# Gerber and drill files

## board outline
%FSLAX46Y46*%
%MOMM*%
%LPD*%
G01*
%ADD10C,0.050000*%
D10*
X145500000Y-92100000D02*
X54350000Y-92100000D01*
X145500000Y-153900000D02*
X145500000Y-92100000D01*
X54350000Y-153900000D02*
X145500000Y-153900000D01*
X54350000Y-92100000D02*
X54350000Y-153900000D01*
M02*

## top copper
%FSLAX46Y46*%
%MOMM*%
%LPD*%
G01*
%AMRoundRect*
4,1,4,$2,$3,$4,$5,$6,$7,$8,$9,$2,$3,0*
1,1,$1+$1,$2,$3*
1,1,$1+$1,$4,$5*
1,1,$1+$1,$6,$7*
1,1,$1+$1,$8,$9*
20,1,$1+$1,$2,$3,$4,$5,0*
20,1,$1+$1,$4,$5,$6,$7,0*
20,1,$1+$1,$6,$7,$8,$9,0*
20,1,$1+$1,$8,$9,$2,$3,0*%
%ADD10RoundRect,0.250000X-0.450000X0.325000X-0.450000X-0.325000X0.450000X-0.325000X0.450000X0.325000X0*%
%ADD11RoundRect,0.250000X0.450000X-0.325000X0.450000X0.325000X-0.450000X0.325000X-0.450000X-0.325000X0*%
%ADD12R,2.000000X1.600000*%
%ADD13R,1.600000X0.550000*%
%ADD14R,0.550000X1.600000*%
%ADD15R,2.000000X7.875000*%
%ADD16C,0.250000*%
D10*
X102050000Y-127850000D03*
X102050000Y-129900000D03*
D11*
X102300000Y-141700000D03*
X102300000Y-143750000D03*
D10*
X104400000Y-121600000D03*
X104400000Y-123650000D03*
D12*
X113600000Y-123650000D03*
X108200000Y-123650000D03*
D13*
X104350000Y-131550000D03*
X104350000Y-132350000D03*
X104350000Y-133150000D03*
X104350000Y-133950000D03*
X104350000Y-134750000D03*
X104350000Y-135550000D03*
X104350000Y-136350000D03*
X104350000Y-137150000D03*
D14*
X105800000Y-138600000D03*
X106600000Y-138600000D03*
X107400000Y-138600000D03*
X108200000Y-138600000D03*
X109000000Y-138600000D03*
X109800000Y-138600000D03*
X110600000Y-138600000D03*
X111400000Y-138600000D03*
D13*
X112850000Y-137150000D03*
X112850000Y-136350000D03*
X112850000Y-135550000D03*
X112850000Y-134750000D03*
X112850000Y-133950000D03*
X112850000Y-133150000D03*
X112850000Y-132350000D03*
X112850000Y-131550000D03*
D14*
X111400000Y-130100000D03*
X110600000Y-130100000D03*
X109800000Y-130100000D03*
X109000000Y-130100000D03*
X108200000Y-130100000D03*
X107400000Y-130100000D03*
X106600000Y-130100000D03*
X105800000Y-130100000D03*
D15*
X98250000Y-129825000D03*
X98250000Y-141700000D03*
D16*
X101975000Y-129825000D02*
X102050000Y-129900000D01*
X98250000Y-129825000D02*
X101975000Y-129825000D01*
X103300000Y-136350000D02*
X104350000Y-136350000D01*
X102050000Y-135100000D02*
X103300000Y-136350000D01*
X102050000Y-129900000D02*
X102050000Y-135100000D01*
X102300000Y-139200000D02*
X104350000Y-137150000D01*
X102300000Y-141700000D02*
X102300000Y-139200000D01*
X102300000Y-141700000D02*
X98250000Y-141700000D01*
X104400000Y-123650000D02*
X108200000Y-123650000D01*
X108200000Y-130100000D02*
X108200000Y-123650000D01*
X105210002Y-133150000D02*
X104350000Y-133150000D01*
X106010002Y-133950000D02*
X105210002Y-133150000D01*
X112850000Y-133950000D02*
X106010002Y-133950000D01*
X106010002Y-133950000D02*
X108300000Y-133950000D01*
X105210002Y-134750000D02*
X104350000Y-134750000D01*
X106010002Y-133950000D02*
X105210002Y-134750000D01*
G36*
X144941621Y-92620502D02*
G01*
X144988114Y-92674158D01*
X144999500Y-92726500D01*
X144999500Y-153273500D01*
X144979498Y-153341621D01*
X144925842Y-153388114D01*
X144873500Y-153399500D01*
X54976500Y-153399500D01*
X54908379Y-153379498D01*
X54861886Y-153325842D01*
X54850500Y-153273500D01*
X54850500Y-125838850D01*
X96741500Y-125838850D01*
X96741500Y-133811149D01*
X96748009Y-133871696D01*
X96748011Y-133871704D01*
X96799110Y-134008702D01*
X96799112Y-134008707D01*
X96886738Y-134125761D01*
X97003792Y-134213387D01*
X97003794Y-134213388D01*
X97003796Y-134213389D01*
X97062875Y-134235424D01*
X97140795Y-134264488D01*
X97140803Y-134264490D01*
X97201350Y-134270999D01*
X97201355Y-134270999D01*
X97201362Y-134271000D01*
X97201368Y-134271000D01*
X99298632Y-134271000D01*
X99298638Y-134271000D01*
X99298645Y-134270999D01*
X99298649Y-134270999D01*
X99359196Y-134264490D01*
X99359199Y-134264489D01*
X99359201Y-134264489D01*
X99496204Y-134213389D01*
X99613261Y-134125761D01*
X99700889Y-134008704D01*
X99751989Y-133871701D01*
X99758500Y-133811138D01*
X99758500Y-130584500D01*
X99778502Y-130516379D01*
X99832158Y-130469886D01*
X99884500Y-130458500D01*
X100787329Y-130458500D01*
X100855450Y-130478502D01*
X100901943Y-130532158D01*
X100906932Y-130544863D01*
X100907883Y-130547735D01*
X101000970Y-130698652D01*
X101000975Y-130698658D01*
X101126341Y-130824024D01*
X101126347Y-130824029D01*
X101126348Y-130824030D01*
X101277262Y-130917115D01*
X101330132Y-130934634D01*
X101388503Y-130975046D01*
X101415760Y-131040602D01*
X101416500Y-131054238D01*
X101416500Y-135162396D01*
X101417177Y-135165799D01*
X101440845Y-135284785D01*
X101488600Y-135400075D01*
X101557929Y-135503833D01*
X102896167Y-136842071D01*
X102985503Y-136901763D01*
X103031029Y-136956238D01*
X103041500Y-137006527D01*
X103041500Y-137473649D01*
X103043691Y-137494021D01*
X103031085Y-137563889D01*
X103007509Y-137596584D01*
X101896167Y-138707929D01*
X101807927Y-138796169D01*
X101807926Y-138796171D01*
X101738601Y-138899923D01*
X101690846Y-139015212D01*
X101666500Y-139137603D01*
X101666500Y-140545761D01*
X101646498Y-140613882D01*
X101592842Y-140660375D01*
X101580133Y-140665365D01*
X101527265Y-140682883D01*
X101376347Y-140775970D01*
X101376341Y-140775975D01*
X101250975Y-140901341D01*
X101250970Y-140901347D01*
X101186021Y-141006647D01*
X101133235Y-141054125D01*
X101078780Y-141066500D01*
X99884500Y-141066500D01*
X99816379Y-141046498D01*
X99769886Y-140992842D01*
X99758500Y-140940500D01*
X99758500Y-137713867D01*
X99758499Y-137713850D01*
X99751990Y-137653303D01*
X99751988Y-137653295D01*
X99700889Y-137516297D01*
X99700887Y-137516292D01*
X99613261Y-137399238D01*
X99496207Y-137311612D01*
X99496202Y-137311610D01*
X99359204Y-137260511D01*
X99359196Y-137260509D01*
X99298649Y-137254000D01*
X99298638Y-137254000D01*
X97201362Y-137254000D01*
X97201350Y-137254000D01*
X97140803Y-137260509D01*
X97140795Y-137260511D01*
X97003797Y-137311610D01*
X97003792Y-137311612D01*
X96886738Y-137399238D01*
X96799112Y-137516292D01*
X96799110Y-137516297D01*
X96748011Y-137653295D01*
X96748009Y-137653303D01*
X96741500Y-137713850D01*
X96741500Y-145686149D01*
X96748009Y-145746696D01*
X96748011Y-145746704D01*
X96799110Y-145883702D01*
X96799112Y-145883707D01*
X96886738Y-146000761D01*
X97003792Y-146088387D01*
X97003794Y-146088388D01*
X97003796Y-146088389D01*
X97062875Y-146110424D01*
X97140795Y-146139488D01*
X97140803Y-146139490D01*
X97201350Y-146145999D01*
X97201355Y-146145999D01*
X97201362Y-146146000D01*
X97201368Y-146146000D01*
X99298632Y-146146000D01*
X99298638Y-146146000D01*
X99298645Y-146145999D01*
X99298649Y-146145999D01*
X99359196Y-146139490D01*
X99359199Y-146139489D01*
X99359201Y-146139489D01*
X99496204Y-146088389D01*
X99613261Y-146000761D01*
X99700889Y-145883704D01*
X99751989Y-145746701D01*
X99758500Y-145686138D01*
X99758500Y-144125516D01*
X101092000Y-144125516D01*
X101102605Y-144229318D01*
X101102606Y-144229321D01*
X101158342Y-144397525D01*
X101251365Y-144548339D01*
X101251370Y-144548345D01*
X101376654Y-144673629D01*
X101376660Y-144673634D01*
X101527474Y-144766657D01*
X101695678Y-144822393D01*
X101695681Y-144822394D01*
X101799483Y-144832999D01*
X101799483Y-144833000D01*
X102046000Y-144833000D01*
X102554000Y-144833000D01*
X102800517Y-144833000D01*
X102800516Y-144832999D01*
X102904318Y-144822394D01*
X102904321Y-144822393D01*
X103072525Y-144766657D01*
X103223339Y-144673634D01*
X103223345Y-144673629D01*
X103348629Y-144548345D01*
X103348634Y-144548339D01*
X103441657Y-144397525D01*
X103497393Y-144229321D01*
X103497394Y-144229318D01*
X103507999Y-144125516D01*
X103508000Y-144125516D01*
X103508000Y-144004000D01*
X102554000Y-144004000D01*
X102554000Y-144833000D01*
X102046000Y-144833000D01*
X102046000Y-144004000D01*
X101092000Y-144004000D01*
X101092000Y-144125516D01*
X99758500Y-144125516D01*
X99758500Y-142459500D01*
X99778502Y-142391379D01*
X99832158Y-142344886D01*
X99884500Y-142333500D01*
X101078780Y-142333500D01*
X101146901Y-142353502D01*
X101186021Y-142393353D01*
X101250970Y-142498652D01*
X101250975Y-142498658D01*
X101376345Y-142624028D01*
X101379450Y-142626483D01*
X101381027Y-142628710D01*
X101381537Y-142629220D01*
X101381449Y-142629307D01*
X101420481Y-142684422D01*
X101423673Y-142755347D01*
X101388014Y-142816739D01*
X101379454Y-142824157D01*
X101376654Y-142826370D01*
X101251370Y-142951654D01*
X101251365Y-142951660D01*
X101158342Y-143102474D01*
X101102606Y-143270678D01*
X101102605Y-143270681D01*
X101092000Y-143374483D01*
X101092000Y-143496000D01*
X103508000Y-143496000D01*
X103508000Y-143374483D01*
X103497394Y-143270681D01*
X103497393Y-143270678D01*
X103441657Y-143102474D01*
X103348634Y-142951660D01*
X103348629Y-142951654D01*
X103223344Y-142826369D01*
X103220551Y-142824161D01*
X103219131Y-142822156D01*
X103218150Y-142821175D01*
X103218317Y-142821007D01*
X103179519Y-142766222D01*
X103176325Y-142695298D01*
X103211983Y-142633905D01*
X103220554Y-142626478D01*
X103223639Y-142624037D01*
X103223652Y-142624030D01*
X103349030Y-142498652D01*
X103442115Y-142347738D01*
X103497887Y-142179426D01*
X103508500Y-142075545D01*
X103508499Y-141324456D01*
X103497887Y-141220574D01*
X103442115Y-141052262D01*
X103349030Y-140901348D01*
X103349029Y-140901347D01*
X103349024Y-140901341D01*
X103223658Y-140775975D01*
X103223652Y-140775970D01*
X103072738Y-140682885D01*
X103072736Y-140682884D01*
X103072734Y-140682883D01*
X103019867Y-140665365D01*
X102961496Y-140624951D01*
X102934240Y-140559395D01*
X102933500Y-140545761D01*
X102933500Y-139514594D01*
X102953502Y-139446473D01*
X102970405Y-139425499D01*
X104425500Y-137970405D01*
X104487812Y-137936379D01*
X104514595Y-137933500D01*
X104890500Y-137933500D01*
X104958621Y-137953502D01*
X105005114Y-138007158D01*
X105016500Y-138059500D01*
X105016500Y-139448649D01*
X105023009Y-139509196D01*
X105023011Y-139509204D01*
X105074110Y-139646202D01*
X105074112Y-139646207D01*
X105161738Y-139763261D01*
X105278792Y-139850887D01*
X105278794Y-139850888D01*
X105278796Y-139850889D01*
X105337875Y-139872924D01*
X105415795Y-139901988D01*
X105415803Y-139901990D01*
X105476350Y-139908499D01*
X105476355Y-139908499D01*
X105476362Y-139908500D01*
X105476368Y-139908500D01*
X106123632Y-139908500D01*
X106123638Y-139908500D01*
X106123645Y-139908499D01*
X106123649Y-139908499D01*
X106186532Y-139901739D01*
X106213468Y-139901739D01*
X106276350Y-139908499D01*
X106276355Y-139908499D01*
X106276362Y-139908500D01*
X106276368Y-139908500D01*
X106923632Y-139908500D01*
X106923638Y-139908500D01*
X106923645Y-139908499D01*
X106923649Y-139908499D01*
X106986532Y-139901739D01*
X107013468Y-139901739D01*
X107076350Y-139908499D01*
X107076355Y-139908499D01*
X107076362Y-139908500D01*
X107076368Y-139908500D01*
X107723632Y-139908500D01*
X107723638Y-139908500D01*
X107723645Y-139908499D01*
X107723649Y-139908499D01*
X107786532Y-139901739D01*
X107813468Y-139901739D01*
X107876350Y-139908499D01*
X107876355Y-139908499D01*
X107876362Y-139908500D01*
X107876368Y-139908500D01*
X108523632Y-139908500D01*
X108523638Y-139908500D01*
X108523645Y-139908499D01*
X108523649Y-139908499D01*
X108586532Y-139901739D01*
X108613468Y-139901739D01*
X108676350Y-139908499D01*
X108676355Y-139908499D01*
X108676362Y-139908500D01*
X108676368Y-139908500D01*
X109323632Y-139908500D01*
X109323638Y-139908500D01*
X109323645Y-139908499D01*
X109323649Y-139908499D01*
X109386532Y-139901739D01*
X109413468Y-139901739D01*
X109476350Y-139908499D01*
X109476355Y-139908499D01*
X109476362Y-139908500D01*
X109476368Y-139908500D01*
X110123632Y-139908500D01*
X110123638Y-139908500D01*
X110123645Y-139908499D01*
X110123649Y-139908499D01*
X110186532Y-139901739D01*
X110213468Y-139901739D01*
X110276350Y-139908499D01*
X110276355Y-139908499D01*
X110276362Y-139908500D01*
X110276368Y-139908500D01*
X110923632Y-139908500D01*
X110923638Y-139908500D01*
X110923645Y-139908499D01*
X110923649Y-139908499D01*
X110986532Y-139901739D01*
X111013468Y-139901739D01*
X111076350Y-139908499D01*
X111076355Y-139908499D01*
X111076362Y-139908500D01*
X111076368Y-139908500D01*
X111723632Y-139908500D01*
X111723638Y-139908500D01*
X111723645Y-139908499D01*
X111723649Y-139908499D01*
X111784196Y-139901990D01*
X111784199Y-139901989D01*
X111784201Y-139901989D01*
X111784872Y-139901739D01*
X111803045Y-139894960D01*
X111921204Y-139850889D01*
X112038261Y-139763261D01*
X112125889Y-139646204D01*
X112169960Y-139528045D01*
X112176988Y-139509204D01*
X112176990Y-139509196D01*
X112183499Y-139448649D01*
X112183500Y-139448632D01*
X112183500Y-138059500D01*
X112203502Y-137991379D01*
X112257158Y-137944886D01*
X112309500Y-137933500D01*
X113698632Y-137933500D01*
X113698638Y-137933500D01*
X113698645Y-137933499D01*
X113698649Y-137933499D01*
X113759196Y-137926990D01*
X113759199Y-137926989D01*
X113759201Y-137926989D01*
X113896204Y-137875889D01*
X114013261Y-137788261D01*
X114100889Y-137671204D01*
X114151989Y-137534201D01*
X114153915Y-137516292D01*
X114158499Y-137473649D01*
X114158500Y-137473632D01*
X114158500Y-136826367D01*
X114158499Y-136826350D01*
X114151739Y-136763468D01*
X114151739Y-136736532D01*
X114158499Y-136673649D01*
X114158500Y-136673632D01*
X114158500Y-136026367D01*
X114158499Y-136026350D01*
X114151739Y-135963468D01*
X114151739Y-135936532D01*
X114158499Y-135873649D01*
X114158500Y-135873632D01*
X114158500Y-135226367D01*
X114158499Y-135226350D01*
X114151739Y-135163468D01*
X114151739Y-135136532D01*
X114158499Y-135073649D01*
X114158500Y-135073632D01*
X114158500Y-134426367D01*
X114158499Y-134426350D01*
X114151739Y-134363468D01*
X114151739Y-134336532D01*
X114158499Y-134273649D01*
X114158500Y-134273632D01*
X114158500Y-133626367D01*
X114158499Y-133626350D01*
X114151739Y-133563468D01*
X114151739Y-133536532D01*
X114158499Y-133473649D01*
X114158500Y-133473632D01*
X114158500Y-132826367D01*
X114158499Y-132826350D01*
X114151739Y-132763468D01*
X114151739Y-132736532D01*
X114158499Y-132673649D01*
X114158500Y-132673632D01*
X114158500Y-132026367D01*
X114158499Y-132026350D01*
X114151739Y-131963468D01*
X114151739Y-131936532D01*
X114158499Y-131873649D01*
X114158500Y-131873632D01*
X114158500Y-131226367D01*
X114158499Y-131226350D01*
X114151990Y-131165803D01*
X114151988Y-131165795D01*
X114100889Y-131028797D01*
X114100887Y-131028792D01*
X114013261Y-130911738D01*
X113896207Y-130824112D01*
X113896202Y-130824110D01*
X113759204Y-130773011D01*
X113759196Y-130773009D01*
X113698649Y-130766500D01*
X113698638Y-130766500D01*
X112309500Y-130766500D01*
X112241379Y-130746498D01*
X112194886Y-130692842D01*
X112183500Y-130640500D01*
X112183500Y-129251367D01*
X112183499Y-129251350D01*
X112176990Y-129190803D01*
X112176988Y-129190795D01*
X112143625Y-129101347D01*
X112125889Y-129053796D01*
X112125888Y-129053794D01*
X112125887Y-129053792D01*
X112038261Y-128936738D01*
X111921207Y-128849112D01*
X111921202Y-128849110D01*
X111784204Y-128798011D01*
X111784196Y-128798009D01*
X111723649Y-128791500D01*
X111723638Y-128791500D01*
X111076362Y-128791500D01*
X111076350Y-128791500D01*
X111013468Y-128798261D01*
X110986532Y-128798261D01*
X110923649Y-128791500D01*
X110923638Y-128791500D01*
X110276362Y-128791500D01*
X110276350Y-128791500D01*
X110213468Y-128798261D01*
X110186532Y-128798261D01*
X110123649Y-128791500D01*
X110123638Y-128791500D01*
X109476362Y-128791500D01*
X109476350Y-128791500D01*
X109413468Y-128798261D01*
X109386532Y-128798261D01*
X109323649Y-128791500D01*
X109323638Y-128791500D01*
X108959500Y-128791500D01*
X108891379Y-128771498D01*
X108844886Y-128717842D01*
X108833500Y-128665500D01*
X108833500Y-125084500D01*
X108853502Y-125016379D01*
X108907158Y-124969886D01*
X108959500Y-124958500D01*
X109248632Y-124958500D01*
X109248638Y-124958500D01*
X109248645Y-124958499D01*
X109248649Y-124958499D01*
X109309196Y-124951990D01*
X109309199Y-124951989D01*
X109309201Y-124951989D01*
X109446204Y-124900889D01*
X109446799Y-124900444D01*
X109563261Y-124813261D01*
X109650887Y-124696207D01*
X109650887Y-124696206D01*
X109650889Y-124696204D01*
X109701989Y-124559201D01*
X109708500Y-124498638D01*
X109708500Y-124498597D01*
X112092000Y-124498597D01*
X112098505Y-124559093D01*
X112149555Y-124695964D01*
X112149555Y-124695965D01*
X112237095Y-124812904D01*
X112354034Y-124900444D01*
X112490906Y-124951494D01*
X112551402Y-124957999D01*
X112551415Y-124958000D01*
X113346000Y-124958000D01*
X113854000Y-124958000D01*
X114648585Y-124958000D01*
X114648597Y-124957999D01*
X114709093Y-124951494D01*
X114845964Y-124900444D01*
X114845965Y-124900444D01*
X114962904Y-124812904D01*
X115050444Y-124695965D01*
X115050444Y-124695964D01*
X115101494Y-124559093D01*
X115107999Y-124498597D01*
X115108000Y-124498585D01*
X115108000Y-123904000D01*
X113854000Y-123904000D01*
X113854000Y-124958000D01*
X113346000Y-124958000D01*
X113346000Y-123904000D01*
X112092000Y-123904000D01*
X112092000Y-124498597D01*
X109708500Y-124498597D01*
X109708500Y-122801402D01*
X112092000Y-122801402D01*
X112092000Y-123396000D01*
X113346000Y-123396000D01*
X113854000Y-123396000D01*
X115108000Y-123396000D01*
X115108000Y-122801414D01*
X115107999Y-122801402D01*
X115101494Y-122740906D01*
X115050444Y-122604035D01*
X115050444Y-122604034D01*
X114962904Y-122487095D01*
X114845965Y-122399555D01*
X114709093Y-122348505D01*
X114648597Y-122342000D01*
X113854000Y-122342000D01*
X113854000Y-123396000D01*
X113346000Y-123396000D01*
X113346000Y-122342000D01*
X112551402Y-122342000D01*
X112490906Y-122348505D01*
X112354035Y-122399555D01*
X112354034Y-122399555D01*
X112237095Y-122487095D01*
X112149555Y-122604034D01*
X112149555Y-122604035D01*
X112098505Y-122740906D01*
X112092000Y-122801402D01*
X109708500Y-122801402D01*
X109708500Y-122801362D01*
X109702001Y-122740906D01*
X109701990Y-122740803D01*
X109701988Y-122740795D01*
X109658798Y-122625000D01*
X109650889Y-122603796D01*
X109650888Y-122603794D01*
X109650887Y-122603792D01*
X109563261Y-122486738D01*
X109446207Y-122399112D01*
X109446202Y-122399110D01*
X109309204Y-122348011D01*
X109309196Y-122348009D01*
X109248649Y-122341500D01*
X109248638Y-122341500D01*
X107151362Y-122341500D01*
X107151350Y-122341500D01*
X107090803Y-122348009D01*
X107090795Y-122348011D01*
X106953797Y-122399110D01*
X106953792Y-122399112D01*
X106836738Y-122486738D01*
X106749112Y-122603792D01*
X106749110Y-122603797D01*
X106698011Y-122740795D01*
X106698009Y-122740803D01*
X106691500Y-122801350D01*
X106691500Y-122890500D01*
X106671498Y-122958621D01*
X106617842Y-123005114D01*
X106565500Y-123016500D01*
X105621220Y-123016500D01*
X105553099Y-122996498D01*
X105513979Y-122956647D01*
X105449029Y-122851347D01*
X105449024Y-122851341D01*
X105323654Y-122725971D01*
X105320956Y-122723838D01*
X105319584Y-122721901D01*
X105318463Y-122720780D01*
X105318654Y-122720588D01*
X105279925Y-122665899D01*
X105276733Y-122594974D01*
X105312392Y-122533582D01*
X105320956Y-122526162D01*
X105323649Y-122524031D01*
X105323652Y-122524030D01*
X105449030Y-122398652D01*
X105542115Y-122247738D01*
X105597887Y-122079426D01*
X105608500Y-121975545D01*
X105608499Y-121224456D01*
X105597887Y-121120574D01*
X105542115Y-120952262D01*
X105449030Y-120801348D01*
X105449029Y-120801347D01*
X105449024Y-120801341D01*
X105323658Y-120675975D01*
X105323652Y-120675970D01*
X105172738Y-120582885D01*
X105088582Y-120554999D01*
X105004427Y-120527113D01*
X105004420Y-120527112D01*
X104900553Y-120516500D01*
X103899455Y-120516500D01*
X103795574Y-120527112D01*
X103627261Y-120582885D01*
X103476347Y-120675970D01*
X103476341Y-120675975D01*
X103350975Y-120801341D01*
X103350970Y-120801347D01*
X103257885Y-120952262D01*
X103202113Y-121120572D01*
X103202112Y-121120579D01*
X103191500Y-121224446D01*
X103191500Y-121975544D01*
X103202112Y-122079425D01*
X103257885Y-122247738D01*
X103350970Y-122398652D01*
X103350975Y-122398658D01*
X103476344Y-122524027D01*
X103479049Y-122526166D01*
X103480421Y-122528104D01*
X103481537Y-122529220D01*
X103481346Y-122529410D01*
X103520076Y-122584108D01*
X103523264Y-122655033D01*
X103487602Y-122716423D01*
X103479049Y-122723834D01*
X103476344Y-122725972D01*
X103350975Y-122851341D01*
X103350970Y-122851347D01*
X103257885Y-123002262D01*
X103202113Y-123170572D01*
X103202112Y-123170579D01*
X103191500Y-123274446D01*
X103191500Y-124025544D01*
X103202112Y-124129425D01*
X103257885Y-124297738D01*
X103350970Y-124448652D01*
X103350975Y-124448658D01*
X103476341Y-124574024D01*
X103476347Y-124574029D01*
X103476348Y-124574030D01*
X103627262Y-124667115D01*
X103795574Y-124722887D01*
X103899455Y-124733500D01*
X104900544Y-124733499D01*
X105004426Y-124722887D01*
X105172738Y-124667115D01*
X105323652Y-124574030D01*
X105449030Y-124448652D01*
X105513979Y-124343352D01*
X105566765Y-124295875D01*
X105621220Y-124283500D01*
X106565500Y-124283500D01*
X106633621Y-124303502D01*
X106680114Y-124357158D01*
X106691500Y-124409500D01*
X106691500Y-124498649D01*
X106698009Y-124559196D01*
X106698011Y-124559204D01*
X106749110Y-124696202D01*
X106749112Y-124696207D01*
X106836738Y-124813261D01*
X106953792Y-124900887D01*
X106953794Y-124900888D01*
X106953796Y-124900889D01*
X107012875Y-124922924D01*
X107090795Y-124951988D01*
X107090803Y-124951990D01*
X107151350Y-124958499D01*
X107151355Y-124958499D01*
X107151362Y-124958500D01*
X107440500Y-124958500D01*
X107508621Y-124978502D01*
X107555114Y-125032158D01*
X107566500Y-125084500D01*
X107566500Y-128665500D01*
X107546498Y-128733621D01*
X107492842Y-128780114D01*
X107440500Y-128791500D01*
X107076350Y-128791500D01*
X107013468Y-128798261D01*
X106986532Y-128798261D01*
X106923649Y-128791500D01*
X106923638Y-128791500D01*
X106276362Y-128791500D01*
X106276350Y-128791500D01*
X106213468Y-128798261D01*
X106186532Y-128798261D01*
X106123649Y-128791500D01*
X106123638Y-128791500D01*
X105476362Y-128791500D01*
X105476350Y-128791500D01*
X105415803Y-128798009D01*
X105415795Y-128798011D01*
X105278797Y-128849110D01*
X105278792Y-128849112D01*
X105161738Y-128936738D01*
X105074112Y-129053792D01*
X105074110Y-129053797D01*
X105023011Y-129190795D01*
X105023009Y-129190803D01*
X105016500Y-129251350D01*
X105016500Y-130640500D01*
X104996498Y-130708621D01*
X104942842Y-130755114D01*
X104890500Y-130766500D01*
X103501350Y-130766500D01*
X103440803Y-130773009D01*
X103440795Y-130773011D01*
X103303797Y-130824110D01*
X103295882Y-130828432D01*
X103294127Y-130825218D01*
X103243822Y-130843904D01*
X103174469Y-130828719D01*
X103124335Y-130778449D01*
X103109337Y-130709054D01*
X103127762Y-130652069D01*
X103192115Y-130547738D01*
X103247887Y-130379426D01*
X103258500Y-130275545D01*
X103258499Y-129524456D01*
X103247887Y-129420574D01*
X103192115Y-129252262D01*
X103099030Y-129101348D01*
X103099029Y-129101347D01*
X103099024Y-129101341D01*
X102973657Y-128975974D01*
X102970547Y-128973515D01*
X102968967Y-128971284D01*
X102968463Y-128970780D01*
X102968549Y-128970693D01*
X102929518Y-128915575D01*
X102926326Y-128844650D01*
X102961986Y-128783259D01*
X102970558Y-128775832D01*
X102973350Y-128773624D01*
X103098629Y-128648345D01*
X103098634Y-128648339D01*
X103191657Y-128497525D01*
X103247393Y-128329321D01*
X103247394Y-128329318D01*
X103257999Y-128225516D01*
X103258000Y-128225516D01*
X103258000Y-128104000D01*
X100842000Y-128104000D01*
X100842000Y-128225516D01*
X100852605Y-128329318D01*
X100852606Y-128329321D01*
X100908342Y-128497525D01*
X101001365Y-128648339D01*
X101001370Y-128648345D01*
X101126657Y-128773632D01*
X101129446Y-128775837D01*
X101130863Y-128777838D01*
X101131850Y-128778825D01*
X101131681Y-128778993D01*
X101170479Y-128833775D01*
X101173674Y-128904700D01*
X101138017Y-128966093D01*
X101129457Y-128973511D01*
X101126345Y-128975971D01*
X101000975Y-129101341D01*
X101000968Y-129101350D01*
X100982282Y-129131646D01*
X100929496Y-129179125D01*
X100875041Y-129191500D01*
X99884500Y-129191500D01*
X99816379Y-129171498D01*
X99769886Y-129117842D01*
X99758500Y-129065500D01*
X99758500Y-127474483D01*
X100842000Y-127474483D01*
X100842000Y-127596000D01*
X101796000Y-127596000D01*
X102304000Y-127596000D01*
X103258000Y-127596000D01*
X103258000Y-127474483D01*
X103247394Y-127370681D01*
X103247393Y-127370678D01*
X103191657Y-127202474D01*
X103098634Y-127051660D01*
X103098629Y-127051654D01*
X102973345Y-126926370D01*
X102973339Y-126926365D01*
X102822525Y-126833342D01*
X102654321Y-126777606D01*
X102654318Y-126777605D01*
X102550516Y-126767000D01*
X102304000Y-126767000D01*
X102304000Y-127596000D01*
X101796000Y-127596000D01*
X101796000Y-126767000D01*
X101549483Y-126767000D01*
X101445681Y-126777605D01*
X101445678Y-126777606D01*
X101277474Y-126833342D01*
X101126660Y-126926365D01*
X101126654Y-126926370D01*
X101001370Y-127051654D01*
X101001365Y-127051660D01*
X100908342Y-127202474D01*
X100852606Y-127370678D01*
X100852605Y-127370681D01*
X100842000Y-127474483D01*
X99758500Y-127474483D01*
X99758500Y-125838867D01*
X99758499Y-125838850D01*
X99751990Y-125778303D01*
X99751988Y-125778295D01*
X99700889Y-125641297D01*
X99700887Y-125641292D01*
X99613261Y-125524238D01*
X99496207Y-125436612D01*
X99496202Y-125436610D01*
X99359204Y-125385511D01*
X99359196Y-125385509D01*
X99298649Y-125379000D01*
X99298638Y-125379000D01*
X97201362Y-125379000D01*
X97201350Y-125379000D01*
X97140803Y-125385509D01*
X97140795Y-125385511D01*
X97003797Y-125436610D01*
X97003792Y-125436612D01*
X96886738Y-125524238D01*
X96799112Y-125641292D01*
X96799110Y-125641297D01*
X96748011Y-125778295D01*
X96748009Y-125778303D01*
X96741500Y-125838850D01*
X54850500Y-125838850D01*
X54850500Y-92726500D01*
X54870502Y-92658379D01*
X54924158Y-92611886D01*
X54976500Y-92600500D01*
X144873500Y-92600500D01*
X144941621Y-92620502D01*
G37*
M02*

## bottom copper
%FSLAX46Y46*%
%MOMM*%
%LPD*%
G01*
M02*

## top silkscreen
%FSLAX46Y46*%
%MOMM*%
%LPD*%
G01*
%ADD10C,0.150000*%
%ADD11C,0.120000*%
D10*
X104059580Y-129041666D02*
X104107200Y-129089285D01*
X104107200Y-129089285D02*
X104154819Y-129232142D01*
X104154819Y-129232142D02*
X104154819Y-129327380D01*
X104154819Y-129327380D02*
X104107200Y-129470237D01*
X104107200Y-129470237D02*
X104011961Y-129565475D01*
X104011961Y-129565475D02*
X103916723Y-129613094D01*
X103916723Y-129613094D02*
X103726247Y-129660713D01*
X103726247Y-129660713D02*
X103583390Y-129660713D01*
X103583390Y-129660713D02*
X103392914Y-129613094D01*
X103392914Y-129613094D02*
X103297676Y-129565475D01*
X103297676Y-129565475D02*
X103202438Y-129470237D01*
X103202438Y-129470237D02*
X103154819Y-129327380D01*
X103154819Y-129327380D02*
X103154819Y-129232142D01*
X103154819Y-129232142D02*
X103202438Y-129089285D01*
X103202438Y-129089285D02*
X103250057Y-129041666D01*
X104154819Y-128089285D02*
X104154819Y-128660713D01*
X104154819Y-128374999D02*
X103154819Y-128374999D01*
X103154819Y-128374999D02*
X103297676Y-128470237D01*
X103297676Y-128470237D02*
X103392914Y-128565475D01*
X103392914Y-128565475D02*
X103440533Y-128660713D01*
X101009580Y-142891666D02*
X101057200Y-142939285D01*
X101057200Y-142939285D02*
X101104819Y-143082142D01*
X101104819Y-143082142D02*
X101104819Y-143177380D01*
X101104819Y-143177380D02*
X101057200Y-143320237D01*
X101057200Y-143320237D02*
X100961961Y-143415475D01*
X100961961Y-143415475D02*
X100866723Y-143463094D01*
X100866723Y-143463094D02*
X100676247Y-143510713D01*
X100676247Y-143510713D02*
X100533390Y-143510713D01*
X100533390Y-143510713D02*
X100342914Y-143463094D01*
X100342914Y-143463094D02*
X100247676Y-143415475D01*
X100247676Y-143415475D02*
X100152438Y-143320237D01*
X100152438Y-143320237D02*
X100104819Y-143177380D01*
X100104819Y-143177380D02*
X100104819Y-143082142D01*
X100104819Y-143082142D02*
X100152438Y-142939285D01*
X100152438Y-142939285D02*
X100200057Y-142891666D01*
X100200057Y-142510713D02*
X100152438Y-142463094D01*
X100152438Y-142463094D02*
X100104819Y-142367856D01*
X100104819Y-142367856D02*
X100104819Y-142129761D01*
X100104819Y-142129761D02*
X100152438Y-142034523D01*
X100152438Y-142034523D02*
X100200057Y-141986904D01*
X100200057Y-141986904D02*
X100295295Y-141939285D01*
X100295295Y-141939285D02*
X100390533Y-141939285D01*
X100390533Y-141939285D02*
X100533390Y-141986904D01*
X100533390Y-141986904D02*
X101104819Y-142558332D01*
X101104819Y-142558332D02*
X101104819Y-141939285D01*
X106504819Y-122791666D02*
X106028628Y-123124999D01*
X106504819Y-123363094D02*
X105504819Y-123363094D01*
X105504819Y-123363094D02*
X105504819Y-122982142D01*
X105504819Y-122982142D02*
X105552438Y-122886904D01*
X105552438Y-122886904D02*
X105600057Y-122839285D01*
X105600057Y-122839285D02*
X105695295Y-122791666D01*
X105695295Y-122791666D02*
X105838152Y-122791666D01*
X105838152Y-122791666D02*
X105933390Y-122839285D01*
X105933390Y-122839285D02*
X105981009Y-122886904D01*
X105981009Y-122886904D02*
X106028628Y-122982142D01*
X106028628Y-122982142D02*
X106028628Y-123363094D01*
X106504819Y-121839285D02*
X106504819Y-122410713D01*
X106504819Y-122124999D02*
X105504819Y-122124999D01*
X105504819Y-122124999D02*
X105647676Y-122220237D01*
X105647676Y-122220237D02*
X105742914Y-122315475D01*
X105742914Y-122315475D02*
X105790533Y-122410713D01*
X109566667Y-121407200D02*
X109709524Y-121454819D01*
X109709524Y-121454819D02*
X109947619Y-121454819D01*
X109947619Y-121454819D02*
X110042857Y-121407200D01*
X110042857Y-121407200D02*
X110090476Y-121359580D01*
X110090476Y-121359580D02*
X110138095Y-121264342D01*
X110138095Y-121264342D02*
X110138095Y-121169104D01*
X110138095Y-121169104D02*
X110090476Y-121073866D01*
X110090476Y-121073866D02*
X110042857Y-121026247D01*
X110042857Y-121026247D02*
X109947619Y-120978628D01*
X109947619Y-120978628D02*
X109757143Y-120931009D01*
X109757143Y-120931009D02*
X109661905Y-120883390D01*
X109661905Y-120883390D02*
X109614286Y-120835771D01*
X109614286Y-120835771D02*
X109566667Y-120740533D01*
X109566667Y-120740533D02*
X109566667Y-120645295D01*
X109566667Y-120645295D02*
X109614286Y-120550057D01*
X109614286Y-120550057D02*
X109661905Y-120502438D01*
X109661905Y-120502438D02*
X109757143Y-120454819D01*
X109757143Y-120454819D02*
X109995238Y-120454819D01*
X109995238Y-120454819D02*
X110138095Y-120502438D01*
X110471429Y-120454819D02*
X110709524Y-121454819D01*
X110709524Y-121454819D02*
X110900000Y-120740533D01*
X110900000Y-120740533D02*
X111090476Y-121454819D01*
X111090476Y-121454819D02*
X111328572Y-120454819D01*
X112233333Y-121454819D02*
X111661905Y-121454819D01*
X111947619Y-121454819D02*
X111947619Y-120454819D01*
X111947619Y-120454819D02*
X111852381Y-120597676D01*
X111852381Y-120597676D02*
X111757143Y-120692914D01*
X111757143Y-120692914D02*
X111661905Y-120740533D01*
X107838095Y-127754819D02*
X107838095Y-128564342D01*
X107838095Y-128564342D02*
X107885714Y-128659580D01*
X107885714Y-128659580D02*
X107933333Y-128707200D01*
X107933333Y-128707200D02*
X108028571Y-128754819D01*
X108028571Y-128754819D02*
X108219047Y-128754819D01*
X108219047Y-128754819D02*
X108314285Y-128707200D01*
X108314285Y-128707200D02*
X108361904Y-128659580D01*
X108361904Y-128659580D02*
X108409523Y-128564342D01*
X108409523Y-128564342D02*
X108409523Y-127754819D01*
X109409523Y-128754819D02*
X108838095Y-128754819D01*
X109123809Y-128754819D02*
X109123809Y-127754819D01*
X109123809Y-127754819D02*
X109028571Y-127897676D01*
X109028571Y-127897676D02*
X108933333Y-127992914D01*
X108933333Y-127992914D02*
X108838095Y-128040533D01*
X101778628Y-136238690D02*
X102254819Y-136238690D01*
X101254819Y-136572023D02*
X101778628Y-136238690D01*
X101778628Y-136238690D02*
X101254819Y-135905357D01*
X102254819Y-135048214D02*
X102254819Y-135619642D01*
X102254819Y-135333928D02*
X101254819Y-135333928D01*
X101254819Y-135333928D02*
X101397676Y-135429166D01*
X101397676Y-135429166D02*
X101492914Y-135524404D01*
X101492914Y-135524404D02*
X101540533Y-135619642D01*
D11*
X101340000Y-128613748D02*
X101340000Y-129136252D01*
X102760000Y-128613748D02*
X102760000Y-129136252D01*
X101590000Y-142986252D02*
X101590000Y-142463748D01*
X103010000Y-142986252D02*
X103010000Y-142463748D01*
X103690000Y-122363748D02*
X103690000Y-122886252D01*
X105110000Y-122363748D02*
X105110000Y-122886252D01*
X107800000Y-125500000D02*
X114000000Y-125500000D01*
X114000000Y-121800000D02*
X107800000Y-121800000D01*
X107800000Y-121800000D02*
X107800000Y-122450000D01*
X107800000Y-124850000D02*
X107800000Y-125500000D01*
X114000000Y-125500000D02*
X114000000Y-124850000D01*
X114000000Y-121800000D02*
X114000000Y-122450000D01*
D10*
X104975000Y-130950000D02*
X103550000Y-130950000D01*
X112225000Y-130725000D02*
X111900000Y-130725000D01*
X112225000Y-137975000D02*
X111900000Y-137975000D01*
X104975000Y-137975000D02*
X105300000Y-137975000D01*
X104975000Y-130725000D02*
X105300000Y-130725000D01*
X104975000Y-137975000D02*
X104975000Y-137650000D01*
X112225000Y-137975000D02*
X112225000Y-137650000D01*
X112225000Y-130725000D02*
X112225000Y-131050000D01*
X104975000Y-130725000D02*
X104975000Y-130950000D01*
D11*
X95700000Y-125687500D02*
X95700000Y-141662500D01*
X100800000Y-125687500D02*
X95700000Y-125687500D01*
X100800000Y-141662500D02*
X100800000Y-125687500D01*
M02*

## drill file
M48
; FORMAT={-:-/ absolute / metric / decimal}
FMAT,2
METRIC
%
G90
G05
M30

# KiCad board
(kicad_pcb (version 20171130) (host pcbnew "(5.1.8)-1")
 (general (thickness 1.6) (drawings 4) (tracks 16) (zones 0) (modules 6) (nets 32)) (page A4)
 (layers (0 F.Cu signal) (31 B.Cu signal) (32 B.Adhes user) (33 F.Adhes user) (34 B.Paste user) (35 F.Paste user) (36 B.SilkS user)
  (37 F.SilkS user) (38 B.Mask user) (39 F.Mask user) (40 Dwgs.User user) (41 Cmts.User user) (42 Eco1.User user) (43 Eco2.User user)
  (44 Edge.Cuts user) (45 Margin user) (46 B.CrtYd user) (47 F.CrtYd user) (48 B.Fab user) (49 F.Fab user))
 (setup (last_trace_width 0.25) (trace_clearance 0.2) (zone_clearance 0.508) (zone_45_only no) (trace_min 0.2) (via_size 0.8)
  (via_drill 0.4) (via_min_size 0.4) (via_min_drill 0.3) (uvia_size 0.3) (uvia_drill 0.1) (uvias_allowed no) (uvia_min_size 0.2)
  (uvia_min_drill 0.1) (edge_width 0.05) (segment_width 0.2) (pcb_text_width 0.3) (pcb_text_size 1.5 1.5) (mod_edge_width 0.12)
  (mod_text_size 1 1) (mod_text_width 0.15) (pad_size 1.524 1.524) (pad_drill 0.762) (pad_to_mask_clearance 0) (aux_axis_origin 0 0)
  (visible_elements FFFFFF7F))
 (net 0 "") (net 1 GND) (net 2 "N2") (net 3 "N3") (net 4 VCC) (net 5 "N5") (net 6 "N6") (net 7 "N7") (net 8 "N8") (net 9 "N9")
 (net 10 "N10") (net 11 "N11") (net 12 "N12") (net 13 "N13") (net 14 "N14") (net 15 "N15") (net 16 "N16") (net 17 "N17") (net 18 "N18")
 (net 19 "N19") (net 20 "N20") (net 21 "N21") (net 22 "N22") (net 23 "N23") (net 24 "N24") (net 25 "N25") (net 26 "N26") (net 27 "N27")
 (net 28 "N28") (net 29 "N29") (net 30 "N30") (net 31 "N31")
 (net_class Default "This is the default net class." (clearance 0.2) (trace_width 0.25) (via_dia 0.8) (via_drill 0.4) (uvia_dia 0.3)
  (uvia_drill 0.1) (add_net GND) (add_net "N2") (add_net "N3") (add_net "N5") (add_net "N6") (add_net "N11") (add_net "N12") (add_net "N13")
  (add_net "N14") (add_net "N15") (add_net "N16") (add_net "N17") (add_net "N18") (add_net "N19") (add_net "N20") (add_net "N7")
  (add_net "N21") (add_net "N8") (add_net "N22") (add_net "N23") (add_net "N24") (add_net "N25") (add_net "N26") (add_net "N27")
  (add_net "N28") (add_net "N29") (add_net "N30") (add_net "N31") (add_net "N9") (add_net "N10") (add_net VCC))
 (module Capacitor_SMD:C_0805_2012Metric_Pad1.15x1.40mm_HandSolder (layer F.Cu) (at 102.05 128.875 270)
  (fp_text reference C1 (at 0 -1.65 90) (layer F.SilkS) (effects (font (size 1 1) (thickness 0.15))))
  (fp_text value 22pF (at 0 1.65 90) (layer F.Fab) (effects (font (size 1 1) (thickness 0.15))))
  (fp_line (start -0.261252 0.71) (end 0.261252 0.71) (layer F.SilkS) (width 0.12))
  (fp_line (start -0.261252 -0.71) (end 0.261252 -0.71) (layer F.SilkS) (width 0.12))
  (pad 1 smd roundrect (at -1.025 0 270) (size 1.15 1.4) (layers F.Cu F.Paste F.Mask) (roundrect_rratio 0.217391) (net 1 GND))
  (pad 2 smd roundrect (at 1.025 0 270) (size 1.15 1.4) (layers F.Cu F.Paste F.Mask) (roundrect_rratio 0.217391) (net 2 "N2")))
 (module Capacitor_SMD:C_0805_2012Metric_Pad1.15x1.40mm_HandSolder (layer F.Cu) (at 102.3 142.725 90)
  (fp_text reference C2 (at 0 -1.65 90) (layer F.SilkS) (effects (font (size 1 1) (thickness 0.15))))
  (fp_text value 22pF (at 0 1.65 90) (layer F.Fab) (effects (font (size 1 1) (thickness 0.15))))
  (fp_line (start -0.261252 -0.71) (end 0.261252 -0.71) (layer F.SilkS) (width 0.12))
  (fp_line (start -0.261252 0.71) (end 0.261252 0.71) (layer F.SilkS) (width 0.12))
  (pad 2 smd roundrect (at 1.025 0 90) (size 1.15 1.4) (layers F.Cu F.Paste F.Mask) (roundrect_rratio 0.217391) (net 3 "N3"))
  (pad 1 smd roundrect (at -1.025 0 90) (size 1.15 1.4) (layers F.Cu F.Paste F.Mask) (roundrect_rratio 0.217391) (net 1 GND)))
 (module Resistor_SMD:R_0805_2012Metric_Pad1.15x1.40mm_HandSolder (layer F.Cu) (at 104.4 122.625 270)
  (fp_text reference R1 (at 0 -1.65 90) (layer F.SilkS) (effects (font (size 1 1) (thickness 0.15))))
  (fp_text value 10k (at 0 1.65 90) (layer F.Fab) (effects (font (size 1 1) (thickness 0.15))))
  (fp_line (start -0.261252 0.71) (end 0.261252 0.71) (layer F.SilkS) (width 0.12))
  (fp_line (start -0.261252 -0.71) (end 0.261252 -0.71) (layer F.SilkS) (width 0.12))
  (pad 1 smd roundrect (at -1.025 0 270) (size 1.15 1.4) (layers F.Cu F.Paste F.Mask) (roundrect_rratio 0.217391) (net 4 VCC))
  (pad 2 smd roundrect (at 1.025 0 270) (size 1.15 1.4) (layers F.Cu F.Paste F.Mask) (roundrect_rratio 0.217391) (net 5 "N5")))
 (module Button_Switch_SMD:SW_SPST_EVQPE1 (layer F.Cu) (at 110.9 123.65)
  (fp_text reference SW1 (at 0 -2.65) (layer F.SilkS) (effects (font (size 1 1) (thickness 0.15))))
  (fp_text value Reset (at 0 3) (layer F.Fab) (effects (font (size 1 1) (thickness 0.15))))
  (fp_line (start -3.1 1.85) (end 3.1 1.85) (layer F.SilkS) (width 0.12))
  (fp_line (start 3.1 -1.85) (end -3.1 -1.85) (layer F.SilkS) (width 0.12))
  (fp_line (start -3.1 -1.85) (end -3.1 -1.2) (layer F.SilkS) (width 0.12))
  (fp_line (start -3.1 1.2) (end -3.1 1.85) (layer F.SilkS) (width 0.12))
  (fp_line (start 3.1 1.85) (end 3.1 1.2) (layer F.SilkS) (width 0.12))
  (fp_line (start 3.1 -1.85) (end 3.1 -1.2) (layer F.SilkS) (width 0.12))
  (pad 2 smd rect (at 2.7 0) (size 2 1.6) (layers F.Cu F.Paste F.Mask) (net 1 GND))
  (pad 1 smd rect (at -2.7 0) (size 2 1.6) (layers F.Cu F.Paste F.Mask) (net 5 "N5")))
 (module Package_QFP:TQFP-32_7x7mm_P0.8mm (layer F.Cu) (at 108.6 134.35)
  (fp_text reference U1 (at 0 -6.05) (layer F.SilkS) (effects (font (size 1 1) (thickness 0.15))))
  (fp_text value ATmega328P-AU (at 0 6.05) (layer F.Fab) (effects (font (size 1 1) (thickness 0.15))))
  (fp_line (start -3.625 -3.4) (end -5.05 -3.4) (layer F.SilkS) (width 0.15))
  (fp_line (start 3.625 -3.625) (end 3.3 -3.625) (layer F.SilkS) (width 0.15))
  (fp_line (start 3.625 3.625) (end 3.3 3.625) (layer F.SilkS) (width 0.15))
  (fp_line (start -3.625 3.625) (end -3.3 3.625) (layer F.SilkS) (width 0.15))
  (fp_line (start -3.625 -3.625) (end -3.3 -3.625) (layer F.SilkS) (width 0.15))
  (fp_line (start -3.625 3.625) (end -3.625 3.3) (layer F.SilkS) (width 0.15))
  (fp_line (start 3.625 3.625) (end 3.625 3.3) (layer F.SilkS) (width 0.15))
  (fp_line (start 3.625 -3.625) (end 3.625 -3.3) (layer F.SilkS) (width 0.15))
  (fp_line (start -3.625 -3.625) (end -3.625 -3.4) (layer F.SilkS) (width 0.15))
  (pad 1 smd rect (at -4.25 -2.8) (size 1.6 0.55) (layers F.Cu F.Paste F.Mask) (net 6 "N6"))
  (pad 2 smd rect (at -4.25 -2) (size 1.6 0.55) (layers F.Cu F.Paste F.Mask) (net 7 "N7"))
  (pad 3 smd rect (at -4.25 -1.2) (size 1.6 0.55) (layers F.Cu F.Paste F.Mask) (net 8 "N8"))
  (pad 4 smd rect (at -4.25 -0.4) (size 1.6 0.55) (layers F.Cu F.Paste F.Mask) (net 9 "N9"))
  (pad 5 smd rect (at -4.25 0.4) (size 1.6 0.55) (layers F.Cu F.Paste F.Mask) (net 8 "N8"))
  (pad 6 smd rect (at -4.25 1.2) (size 1.6 0.55) (layers F.Cu F.Paste F.Mask) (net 9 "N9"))
  (pad 7 smd rect (at -4.25 2) (size 1.6 0.55) (layers F.Cu F.Paste F.Mask) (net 2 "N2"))
  (pad 8 smd rect (at -4.25 2.8) (size 1.6 0.55) (layers F.Cu F.Paste F.Mask) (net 3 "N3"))
  (pad 9 smd rect (at -2.8 4.25 90) (size 1.6 0.55) (layers F.Cu F.Paste F.Mask) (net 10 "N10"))
  (pad 10 smd rect (at -2 4.25 90) (size 1.6 0.55) (layers F.Cu F.Paste F.Mask) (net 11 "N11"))
  (pad 11 smd rect (at -1.2 4.25 90) (size 1.6 0.55) (layers F.Cu F.Paste F.Mask) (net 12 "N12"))
  (pad 12 smd rect (at -0.4 4.25 90) (size 1.6 0.55) (layers F.Cu F.Paste F.Mask) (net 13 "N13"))
  (pad 13 smd rect (at 0.4 4.25 90) (size 1.6 0.55) (layers F.Cu F.Paste F.Mask) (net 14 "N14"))
  (pad 14 smd rect (at 1.2 4.25 90) (size 1.6 0.55) (layers F.Cu F.Paste F.Mask) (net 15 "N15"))
  (pad 15 smd rect (at 2 4.25 90) (size 1.6 0.55) (layers F.Cu F.Paste F.Mask) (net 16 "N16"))
  (pad 16 smd rect (at 2.8 4.25 90) (size 1.6 0.55) (layers F.Cu F.Paste F.Mask) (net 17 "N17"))
  (pad 17 smd rect (at 4.25 2.8) (size 1.6 0.55) (layers F.Cu F.Paste F.Mask) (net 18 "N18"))
  (pad 18 smd rect (at 4.25 2) (size 1.6 0.55) (layers F.Cu F.Paste F.Mask) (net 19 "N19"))
  (pad 19 smd rect (at 4.25 1.2) (size 1.6 0.55) (layers F.Cu F.Paste F.Mask) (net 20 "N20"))
  (pad 20 smd rect (at 4.25 0.4) (size 1.6 0.55) (layers F.Cu F.Paste F.Mask) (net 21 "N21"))
  (pad 21 smd rect (at 4.25 -0.4) (size 1.6 0.55) (layers F.Cu F.Paste F.Mask) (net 8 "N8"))
  (pad 22 smd rect (at 4.25 -1.2) (size 1.6 0.55) (layers F.Cu F.Paste F.Mask) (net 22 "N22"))
  (pad 23 smd rect (at 4.25 -2) (size 1.6 0.55) (layers F.Cu F.Paste F.Mask) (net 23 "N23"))
  (pad 24 smd rect (at 4.25 -2.8) (size 1.6 0.55) (layers F.Cu F.Paste F.Mask) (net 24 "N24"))
  (pad 25 smd rect (at 2.8 -4.25 90) (size 1.6 0.55) (layers F.Cu F.Paste F.Mask) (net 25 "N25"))
  (pad 26 smd rect (at 2 -4.25 90) (size 1.6 0.55) (layers F.Cu F.Paste F.Mask) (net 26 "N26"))
  (pad 27 smd rect (at 1.2 -4.25 90) (size 1.6 0.55) (layers F.Cu F.Paste F.Mask) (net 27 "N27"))
  (pad 28 smd rect (at 0.4 -4.25 90) (size 1.6 0.55) (layers F.Cu F.Paste F.Mask) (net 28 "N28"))
  (pad 29 smd rect (at -0.4 -4.25 90) (size 1.6 0.55) (layers F.Cu F.Paste F.Mask) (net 5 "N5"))
  (pad 30 smd rect (at -1.2 -4.25 90) (size 1.6 0.55) (layers F.Cu F.Paste F.Mask) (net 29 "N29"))
  (pad 31 smd rect (at -2 -4.25 90) (size 1.6 0.55) (layers F.Cu F.Paste F.Mask) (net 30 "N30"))
  (pad 32 smd rect (at -2.8 -4.25 90) (size 1.6 0.55) (layers F.Cu F.Paste F.Mask) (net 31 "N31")))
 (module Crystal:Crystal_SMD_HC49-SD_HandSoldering (layer F.Cu) (at 98.25 135.7625 270)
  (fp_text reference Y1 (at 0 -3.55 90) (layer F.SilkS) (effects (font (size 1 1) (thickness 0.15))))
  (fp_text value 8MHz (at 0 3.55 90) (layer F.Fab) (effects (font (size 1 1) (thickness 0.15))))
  (fp_line (start -10.075 2.55) (end 5.9 2.55) (layer F.SilkS) (width 0.12))
  (fp_line (start -10.075 -2.55) (end -10.075 2.55) (layer F.SilkS) (width 0.12))
  (fp_line (start 5.9 -2.55) (end -10.075 -2.55) (layer F.SilkS) (width 0.12))
  (pad 1 smd rect (at -5.9375 0 270) (size 7.875 2) (layers F.Cu F.Paste F.Mask) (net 2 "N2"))
  (pad 2 smd rect (at 5.9375 0 270) (size 7.875 2) (layers F.Cu F.Paste F.Mask) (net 3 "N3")))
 (gr_line (start 145.5 92.1) (end 54.35 92.1) (layer Edge.Cuts) (width 0.05))
 (gr_line (start 145.5 153.9) (end 145.5 92.1) (layer Edge.Cuts) (width 0.05))
 (gr_line (start 54.35 153.9) (end 145.5 153.9) (layer Edge.Cuts) (width 0.05))
 (gr_line (start 54.35 92.1) (end 54.35 153.9) (layer Edge.Cuts) (width 0.05))
 (segment (start 101.975 129.825) (end 102.05 129.9) (width 0.25) (layer F.Cu) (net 2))
 (segment (start 98.25 129.825) (end 101.975 129.825) (width 0.25) (layer F.Cu) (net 2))
 (segment (start 103.3 136.35) (end 104.35 136.35) (width 0.25) (layer F.Cu) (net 2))
 (segment (start 102.05 135.1) (end 103.3 136.35) (width 0.25) (layer F.Cu) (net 2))
 (segment (start 102.05 129.9) (end 102.05 135.1) (width 0.25) (layer F.Cu) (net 2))
 (segment (start 102.3 139.2) (end 104.35 137.15) (width 0.25) (layer F.Cu) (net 3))
 (segment (start 102.3 141.7) (end 102.3 139.2) (width 0.25) (layer F.Cu) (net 3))
 (segment (start 102.3 141.7) (end 98.25 141.7) (width 0.25) (layer F.Cu) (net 3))
 (segment (start 104.4 123.65) (end 108.2 123.65) (width 0.25) (layer F.Cu) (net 5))
 (segment (start 108.2 130.1) (end 108.2 123.65) (width 0.25) (layer F.Cu) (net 5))
 (segment (start 105.210002 133.15) (end 104.35 133.15) (width 0.25) (layer F.Cu) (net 8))
 (segment (start 106.010002 133.95) (end 105.210002 133.15) (width 0.25) (layer F.Cu) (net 8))
 (segment (start 112.85 133.95) (end 106.010002 133.95) (width 0.25) (layer F.Cu) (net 8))
 (segment (start 106.010002 133.95) (end 108.3 133.95) (width 0.25) (layer F.Cu) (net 8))
 (segment (start 105.210002 134.75) (end 104.35 134.75) (width 0.25) (layer F.Cu) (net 8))
 (segment (start 106.010002 133.95) (end 105.210002 134.75) (width 0.25) (layer F.Cu) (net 8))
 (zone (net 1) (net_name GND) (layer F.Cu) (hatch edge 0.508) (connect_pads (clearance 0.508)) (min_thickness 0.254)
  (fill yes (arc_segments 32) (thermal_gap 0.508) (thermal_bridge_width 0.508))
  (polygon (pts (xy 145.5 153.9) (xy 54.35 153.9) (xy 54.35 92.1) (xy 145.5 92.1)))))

